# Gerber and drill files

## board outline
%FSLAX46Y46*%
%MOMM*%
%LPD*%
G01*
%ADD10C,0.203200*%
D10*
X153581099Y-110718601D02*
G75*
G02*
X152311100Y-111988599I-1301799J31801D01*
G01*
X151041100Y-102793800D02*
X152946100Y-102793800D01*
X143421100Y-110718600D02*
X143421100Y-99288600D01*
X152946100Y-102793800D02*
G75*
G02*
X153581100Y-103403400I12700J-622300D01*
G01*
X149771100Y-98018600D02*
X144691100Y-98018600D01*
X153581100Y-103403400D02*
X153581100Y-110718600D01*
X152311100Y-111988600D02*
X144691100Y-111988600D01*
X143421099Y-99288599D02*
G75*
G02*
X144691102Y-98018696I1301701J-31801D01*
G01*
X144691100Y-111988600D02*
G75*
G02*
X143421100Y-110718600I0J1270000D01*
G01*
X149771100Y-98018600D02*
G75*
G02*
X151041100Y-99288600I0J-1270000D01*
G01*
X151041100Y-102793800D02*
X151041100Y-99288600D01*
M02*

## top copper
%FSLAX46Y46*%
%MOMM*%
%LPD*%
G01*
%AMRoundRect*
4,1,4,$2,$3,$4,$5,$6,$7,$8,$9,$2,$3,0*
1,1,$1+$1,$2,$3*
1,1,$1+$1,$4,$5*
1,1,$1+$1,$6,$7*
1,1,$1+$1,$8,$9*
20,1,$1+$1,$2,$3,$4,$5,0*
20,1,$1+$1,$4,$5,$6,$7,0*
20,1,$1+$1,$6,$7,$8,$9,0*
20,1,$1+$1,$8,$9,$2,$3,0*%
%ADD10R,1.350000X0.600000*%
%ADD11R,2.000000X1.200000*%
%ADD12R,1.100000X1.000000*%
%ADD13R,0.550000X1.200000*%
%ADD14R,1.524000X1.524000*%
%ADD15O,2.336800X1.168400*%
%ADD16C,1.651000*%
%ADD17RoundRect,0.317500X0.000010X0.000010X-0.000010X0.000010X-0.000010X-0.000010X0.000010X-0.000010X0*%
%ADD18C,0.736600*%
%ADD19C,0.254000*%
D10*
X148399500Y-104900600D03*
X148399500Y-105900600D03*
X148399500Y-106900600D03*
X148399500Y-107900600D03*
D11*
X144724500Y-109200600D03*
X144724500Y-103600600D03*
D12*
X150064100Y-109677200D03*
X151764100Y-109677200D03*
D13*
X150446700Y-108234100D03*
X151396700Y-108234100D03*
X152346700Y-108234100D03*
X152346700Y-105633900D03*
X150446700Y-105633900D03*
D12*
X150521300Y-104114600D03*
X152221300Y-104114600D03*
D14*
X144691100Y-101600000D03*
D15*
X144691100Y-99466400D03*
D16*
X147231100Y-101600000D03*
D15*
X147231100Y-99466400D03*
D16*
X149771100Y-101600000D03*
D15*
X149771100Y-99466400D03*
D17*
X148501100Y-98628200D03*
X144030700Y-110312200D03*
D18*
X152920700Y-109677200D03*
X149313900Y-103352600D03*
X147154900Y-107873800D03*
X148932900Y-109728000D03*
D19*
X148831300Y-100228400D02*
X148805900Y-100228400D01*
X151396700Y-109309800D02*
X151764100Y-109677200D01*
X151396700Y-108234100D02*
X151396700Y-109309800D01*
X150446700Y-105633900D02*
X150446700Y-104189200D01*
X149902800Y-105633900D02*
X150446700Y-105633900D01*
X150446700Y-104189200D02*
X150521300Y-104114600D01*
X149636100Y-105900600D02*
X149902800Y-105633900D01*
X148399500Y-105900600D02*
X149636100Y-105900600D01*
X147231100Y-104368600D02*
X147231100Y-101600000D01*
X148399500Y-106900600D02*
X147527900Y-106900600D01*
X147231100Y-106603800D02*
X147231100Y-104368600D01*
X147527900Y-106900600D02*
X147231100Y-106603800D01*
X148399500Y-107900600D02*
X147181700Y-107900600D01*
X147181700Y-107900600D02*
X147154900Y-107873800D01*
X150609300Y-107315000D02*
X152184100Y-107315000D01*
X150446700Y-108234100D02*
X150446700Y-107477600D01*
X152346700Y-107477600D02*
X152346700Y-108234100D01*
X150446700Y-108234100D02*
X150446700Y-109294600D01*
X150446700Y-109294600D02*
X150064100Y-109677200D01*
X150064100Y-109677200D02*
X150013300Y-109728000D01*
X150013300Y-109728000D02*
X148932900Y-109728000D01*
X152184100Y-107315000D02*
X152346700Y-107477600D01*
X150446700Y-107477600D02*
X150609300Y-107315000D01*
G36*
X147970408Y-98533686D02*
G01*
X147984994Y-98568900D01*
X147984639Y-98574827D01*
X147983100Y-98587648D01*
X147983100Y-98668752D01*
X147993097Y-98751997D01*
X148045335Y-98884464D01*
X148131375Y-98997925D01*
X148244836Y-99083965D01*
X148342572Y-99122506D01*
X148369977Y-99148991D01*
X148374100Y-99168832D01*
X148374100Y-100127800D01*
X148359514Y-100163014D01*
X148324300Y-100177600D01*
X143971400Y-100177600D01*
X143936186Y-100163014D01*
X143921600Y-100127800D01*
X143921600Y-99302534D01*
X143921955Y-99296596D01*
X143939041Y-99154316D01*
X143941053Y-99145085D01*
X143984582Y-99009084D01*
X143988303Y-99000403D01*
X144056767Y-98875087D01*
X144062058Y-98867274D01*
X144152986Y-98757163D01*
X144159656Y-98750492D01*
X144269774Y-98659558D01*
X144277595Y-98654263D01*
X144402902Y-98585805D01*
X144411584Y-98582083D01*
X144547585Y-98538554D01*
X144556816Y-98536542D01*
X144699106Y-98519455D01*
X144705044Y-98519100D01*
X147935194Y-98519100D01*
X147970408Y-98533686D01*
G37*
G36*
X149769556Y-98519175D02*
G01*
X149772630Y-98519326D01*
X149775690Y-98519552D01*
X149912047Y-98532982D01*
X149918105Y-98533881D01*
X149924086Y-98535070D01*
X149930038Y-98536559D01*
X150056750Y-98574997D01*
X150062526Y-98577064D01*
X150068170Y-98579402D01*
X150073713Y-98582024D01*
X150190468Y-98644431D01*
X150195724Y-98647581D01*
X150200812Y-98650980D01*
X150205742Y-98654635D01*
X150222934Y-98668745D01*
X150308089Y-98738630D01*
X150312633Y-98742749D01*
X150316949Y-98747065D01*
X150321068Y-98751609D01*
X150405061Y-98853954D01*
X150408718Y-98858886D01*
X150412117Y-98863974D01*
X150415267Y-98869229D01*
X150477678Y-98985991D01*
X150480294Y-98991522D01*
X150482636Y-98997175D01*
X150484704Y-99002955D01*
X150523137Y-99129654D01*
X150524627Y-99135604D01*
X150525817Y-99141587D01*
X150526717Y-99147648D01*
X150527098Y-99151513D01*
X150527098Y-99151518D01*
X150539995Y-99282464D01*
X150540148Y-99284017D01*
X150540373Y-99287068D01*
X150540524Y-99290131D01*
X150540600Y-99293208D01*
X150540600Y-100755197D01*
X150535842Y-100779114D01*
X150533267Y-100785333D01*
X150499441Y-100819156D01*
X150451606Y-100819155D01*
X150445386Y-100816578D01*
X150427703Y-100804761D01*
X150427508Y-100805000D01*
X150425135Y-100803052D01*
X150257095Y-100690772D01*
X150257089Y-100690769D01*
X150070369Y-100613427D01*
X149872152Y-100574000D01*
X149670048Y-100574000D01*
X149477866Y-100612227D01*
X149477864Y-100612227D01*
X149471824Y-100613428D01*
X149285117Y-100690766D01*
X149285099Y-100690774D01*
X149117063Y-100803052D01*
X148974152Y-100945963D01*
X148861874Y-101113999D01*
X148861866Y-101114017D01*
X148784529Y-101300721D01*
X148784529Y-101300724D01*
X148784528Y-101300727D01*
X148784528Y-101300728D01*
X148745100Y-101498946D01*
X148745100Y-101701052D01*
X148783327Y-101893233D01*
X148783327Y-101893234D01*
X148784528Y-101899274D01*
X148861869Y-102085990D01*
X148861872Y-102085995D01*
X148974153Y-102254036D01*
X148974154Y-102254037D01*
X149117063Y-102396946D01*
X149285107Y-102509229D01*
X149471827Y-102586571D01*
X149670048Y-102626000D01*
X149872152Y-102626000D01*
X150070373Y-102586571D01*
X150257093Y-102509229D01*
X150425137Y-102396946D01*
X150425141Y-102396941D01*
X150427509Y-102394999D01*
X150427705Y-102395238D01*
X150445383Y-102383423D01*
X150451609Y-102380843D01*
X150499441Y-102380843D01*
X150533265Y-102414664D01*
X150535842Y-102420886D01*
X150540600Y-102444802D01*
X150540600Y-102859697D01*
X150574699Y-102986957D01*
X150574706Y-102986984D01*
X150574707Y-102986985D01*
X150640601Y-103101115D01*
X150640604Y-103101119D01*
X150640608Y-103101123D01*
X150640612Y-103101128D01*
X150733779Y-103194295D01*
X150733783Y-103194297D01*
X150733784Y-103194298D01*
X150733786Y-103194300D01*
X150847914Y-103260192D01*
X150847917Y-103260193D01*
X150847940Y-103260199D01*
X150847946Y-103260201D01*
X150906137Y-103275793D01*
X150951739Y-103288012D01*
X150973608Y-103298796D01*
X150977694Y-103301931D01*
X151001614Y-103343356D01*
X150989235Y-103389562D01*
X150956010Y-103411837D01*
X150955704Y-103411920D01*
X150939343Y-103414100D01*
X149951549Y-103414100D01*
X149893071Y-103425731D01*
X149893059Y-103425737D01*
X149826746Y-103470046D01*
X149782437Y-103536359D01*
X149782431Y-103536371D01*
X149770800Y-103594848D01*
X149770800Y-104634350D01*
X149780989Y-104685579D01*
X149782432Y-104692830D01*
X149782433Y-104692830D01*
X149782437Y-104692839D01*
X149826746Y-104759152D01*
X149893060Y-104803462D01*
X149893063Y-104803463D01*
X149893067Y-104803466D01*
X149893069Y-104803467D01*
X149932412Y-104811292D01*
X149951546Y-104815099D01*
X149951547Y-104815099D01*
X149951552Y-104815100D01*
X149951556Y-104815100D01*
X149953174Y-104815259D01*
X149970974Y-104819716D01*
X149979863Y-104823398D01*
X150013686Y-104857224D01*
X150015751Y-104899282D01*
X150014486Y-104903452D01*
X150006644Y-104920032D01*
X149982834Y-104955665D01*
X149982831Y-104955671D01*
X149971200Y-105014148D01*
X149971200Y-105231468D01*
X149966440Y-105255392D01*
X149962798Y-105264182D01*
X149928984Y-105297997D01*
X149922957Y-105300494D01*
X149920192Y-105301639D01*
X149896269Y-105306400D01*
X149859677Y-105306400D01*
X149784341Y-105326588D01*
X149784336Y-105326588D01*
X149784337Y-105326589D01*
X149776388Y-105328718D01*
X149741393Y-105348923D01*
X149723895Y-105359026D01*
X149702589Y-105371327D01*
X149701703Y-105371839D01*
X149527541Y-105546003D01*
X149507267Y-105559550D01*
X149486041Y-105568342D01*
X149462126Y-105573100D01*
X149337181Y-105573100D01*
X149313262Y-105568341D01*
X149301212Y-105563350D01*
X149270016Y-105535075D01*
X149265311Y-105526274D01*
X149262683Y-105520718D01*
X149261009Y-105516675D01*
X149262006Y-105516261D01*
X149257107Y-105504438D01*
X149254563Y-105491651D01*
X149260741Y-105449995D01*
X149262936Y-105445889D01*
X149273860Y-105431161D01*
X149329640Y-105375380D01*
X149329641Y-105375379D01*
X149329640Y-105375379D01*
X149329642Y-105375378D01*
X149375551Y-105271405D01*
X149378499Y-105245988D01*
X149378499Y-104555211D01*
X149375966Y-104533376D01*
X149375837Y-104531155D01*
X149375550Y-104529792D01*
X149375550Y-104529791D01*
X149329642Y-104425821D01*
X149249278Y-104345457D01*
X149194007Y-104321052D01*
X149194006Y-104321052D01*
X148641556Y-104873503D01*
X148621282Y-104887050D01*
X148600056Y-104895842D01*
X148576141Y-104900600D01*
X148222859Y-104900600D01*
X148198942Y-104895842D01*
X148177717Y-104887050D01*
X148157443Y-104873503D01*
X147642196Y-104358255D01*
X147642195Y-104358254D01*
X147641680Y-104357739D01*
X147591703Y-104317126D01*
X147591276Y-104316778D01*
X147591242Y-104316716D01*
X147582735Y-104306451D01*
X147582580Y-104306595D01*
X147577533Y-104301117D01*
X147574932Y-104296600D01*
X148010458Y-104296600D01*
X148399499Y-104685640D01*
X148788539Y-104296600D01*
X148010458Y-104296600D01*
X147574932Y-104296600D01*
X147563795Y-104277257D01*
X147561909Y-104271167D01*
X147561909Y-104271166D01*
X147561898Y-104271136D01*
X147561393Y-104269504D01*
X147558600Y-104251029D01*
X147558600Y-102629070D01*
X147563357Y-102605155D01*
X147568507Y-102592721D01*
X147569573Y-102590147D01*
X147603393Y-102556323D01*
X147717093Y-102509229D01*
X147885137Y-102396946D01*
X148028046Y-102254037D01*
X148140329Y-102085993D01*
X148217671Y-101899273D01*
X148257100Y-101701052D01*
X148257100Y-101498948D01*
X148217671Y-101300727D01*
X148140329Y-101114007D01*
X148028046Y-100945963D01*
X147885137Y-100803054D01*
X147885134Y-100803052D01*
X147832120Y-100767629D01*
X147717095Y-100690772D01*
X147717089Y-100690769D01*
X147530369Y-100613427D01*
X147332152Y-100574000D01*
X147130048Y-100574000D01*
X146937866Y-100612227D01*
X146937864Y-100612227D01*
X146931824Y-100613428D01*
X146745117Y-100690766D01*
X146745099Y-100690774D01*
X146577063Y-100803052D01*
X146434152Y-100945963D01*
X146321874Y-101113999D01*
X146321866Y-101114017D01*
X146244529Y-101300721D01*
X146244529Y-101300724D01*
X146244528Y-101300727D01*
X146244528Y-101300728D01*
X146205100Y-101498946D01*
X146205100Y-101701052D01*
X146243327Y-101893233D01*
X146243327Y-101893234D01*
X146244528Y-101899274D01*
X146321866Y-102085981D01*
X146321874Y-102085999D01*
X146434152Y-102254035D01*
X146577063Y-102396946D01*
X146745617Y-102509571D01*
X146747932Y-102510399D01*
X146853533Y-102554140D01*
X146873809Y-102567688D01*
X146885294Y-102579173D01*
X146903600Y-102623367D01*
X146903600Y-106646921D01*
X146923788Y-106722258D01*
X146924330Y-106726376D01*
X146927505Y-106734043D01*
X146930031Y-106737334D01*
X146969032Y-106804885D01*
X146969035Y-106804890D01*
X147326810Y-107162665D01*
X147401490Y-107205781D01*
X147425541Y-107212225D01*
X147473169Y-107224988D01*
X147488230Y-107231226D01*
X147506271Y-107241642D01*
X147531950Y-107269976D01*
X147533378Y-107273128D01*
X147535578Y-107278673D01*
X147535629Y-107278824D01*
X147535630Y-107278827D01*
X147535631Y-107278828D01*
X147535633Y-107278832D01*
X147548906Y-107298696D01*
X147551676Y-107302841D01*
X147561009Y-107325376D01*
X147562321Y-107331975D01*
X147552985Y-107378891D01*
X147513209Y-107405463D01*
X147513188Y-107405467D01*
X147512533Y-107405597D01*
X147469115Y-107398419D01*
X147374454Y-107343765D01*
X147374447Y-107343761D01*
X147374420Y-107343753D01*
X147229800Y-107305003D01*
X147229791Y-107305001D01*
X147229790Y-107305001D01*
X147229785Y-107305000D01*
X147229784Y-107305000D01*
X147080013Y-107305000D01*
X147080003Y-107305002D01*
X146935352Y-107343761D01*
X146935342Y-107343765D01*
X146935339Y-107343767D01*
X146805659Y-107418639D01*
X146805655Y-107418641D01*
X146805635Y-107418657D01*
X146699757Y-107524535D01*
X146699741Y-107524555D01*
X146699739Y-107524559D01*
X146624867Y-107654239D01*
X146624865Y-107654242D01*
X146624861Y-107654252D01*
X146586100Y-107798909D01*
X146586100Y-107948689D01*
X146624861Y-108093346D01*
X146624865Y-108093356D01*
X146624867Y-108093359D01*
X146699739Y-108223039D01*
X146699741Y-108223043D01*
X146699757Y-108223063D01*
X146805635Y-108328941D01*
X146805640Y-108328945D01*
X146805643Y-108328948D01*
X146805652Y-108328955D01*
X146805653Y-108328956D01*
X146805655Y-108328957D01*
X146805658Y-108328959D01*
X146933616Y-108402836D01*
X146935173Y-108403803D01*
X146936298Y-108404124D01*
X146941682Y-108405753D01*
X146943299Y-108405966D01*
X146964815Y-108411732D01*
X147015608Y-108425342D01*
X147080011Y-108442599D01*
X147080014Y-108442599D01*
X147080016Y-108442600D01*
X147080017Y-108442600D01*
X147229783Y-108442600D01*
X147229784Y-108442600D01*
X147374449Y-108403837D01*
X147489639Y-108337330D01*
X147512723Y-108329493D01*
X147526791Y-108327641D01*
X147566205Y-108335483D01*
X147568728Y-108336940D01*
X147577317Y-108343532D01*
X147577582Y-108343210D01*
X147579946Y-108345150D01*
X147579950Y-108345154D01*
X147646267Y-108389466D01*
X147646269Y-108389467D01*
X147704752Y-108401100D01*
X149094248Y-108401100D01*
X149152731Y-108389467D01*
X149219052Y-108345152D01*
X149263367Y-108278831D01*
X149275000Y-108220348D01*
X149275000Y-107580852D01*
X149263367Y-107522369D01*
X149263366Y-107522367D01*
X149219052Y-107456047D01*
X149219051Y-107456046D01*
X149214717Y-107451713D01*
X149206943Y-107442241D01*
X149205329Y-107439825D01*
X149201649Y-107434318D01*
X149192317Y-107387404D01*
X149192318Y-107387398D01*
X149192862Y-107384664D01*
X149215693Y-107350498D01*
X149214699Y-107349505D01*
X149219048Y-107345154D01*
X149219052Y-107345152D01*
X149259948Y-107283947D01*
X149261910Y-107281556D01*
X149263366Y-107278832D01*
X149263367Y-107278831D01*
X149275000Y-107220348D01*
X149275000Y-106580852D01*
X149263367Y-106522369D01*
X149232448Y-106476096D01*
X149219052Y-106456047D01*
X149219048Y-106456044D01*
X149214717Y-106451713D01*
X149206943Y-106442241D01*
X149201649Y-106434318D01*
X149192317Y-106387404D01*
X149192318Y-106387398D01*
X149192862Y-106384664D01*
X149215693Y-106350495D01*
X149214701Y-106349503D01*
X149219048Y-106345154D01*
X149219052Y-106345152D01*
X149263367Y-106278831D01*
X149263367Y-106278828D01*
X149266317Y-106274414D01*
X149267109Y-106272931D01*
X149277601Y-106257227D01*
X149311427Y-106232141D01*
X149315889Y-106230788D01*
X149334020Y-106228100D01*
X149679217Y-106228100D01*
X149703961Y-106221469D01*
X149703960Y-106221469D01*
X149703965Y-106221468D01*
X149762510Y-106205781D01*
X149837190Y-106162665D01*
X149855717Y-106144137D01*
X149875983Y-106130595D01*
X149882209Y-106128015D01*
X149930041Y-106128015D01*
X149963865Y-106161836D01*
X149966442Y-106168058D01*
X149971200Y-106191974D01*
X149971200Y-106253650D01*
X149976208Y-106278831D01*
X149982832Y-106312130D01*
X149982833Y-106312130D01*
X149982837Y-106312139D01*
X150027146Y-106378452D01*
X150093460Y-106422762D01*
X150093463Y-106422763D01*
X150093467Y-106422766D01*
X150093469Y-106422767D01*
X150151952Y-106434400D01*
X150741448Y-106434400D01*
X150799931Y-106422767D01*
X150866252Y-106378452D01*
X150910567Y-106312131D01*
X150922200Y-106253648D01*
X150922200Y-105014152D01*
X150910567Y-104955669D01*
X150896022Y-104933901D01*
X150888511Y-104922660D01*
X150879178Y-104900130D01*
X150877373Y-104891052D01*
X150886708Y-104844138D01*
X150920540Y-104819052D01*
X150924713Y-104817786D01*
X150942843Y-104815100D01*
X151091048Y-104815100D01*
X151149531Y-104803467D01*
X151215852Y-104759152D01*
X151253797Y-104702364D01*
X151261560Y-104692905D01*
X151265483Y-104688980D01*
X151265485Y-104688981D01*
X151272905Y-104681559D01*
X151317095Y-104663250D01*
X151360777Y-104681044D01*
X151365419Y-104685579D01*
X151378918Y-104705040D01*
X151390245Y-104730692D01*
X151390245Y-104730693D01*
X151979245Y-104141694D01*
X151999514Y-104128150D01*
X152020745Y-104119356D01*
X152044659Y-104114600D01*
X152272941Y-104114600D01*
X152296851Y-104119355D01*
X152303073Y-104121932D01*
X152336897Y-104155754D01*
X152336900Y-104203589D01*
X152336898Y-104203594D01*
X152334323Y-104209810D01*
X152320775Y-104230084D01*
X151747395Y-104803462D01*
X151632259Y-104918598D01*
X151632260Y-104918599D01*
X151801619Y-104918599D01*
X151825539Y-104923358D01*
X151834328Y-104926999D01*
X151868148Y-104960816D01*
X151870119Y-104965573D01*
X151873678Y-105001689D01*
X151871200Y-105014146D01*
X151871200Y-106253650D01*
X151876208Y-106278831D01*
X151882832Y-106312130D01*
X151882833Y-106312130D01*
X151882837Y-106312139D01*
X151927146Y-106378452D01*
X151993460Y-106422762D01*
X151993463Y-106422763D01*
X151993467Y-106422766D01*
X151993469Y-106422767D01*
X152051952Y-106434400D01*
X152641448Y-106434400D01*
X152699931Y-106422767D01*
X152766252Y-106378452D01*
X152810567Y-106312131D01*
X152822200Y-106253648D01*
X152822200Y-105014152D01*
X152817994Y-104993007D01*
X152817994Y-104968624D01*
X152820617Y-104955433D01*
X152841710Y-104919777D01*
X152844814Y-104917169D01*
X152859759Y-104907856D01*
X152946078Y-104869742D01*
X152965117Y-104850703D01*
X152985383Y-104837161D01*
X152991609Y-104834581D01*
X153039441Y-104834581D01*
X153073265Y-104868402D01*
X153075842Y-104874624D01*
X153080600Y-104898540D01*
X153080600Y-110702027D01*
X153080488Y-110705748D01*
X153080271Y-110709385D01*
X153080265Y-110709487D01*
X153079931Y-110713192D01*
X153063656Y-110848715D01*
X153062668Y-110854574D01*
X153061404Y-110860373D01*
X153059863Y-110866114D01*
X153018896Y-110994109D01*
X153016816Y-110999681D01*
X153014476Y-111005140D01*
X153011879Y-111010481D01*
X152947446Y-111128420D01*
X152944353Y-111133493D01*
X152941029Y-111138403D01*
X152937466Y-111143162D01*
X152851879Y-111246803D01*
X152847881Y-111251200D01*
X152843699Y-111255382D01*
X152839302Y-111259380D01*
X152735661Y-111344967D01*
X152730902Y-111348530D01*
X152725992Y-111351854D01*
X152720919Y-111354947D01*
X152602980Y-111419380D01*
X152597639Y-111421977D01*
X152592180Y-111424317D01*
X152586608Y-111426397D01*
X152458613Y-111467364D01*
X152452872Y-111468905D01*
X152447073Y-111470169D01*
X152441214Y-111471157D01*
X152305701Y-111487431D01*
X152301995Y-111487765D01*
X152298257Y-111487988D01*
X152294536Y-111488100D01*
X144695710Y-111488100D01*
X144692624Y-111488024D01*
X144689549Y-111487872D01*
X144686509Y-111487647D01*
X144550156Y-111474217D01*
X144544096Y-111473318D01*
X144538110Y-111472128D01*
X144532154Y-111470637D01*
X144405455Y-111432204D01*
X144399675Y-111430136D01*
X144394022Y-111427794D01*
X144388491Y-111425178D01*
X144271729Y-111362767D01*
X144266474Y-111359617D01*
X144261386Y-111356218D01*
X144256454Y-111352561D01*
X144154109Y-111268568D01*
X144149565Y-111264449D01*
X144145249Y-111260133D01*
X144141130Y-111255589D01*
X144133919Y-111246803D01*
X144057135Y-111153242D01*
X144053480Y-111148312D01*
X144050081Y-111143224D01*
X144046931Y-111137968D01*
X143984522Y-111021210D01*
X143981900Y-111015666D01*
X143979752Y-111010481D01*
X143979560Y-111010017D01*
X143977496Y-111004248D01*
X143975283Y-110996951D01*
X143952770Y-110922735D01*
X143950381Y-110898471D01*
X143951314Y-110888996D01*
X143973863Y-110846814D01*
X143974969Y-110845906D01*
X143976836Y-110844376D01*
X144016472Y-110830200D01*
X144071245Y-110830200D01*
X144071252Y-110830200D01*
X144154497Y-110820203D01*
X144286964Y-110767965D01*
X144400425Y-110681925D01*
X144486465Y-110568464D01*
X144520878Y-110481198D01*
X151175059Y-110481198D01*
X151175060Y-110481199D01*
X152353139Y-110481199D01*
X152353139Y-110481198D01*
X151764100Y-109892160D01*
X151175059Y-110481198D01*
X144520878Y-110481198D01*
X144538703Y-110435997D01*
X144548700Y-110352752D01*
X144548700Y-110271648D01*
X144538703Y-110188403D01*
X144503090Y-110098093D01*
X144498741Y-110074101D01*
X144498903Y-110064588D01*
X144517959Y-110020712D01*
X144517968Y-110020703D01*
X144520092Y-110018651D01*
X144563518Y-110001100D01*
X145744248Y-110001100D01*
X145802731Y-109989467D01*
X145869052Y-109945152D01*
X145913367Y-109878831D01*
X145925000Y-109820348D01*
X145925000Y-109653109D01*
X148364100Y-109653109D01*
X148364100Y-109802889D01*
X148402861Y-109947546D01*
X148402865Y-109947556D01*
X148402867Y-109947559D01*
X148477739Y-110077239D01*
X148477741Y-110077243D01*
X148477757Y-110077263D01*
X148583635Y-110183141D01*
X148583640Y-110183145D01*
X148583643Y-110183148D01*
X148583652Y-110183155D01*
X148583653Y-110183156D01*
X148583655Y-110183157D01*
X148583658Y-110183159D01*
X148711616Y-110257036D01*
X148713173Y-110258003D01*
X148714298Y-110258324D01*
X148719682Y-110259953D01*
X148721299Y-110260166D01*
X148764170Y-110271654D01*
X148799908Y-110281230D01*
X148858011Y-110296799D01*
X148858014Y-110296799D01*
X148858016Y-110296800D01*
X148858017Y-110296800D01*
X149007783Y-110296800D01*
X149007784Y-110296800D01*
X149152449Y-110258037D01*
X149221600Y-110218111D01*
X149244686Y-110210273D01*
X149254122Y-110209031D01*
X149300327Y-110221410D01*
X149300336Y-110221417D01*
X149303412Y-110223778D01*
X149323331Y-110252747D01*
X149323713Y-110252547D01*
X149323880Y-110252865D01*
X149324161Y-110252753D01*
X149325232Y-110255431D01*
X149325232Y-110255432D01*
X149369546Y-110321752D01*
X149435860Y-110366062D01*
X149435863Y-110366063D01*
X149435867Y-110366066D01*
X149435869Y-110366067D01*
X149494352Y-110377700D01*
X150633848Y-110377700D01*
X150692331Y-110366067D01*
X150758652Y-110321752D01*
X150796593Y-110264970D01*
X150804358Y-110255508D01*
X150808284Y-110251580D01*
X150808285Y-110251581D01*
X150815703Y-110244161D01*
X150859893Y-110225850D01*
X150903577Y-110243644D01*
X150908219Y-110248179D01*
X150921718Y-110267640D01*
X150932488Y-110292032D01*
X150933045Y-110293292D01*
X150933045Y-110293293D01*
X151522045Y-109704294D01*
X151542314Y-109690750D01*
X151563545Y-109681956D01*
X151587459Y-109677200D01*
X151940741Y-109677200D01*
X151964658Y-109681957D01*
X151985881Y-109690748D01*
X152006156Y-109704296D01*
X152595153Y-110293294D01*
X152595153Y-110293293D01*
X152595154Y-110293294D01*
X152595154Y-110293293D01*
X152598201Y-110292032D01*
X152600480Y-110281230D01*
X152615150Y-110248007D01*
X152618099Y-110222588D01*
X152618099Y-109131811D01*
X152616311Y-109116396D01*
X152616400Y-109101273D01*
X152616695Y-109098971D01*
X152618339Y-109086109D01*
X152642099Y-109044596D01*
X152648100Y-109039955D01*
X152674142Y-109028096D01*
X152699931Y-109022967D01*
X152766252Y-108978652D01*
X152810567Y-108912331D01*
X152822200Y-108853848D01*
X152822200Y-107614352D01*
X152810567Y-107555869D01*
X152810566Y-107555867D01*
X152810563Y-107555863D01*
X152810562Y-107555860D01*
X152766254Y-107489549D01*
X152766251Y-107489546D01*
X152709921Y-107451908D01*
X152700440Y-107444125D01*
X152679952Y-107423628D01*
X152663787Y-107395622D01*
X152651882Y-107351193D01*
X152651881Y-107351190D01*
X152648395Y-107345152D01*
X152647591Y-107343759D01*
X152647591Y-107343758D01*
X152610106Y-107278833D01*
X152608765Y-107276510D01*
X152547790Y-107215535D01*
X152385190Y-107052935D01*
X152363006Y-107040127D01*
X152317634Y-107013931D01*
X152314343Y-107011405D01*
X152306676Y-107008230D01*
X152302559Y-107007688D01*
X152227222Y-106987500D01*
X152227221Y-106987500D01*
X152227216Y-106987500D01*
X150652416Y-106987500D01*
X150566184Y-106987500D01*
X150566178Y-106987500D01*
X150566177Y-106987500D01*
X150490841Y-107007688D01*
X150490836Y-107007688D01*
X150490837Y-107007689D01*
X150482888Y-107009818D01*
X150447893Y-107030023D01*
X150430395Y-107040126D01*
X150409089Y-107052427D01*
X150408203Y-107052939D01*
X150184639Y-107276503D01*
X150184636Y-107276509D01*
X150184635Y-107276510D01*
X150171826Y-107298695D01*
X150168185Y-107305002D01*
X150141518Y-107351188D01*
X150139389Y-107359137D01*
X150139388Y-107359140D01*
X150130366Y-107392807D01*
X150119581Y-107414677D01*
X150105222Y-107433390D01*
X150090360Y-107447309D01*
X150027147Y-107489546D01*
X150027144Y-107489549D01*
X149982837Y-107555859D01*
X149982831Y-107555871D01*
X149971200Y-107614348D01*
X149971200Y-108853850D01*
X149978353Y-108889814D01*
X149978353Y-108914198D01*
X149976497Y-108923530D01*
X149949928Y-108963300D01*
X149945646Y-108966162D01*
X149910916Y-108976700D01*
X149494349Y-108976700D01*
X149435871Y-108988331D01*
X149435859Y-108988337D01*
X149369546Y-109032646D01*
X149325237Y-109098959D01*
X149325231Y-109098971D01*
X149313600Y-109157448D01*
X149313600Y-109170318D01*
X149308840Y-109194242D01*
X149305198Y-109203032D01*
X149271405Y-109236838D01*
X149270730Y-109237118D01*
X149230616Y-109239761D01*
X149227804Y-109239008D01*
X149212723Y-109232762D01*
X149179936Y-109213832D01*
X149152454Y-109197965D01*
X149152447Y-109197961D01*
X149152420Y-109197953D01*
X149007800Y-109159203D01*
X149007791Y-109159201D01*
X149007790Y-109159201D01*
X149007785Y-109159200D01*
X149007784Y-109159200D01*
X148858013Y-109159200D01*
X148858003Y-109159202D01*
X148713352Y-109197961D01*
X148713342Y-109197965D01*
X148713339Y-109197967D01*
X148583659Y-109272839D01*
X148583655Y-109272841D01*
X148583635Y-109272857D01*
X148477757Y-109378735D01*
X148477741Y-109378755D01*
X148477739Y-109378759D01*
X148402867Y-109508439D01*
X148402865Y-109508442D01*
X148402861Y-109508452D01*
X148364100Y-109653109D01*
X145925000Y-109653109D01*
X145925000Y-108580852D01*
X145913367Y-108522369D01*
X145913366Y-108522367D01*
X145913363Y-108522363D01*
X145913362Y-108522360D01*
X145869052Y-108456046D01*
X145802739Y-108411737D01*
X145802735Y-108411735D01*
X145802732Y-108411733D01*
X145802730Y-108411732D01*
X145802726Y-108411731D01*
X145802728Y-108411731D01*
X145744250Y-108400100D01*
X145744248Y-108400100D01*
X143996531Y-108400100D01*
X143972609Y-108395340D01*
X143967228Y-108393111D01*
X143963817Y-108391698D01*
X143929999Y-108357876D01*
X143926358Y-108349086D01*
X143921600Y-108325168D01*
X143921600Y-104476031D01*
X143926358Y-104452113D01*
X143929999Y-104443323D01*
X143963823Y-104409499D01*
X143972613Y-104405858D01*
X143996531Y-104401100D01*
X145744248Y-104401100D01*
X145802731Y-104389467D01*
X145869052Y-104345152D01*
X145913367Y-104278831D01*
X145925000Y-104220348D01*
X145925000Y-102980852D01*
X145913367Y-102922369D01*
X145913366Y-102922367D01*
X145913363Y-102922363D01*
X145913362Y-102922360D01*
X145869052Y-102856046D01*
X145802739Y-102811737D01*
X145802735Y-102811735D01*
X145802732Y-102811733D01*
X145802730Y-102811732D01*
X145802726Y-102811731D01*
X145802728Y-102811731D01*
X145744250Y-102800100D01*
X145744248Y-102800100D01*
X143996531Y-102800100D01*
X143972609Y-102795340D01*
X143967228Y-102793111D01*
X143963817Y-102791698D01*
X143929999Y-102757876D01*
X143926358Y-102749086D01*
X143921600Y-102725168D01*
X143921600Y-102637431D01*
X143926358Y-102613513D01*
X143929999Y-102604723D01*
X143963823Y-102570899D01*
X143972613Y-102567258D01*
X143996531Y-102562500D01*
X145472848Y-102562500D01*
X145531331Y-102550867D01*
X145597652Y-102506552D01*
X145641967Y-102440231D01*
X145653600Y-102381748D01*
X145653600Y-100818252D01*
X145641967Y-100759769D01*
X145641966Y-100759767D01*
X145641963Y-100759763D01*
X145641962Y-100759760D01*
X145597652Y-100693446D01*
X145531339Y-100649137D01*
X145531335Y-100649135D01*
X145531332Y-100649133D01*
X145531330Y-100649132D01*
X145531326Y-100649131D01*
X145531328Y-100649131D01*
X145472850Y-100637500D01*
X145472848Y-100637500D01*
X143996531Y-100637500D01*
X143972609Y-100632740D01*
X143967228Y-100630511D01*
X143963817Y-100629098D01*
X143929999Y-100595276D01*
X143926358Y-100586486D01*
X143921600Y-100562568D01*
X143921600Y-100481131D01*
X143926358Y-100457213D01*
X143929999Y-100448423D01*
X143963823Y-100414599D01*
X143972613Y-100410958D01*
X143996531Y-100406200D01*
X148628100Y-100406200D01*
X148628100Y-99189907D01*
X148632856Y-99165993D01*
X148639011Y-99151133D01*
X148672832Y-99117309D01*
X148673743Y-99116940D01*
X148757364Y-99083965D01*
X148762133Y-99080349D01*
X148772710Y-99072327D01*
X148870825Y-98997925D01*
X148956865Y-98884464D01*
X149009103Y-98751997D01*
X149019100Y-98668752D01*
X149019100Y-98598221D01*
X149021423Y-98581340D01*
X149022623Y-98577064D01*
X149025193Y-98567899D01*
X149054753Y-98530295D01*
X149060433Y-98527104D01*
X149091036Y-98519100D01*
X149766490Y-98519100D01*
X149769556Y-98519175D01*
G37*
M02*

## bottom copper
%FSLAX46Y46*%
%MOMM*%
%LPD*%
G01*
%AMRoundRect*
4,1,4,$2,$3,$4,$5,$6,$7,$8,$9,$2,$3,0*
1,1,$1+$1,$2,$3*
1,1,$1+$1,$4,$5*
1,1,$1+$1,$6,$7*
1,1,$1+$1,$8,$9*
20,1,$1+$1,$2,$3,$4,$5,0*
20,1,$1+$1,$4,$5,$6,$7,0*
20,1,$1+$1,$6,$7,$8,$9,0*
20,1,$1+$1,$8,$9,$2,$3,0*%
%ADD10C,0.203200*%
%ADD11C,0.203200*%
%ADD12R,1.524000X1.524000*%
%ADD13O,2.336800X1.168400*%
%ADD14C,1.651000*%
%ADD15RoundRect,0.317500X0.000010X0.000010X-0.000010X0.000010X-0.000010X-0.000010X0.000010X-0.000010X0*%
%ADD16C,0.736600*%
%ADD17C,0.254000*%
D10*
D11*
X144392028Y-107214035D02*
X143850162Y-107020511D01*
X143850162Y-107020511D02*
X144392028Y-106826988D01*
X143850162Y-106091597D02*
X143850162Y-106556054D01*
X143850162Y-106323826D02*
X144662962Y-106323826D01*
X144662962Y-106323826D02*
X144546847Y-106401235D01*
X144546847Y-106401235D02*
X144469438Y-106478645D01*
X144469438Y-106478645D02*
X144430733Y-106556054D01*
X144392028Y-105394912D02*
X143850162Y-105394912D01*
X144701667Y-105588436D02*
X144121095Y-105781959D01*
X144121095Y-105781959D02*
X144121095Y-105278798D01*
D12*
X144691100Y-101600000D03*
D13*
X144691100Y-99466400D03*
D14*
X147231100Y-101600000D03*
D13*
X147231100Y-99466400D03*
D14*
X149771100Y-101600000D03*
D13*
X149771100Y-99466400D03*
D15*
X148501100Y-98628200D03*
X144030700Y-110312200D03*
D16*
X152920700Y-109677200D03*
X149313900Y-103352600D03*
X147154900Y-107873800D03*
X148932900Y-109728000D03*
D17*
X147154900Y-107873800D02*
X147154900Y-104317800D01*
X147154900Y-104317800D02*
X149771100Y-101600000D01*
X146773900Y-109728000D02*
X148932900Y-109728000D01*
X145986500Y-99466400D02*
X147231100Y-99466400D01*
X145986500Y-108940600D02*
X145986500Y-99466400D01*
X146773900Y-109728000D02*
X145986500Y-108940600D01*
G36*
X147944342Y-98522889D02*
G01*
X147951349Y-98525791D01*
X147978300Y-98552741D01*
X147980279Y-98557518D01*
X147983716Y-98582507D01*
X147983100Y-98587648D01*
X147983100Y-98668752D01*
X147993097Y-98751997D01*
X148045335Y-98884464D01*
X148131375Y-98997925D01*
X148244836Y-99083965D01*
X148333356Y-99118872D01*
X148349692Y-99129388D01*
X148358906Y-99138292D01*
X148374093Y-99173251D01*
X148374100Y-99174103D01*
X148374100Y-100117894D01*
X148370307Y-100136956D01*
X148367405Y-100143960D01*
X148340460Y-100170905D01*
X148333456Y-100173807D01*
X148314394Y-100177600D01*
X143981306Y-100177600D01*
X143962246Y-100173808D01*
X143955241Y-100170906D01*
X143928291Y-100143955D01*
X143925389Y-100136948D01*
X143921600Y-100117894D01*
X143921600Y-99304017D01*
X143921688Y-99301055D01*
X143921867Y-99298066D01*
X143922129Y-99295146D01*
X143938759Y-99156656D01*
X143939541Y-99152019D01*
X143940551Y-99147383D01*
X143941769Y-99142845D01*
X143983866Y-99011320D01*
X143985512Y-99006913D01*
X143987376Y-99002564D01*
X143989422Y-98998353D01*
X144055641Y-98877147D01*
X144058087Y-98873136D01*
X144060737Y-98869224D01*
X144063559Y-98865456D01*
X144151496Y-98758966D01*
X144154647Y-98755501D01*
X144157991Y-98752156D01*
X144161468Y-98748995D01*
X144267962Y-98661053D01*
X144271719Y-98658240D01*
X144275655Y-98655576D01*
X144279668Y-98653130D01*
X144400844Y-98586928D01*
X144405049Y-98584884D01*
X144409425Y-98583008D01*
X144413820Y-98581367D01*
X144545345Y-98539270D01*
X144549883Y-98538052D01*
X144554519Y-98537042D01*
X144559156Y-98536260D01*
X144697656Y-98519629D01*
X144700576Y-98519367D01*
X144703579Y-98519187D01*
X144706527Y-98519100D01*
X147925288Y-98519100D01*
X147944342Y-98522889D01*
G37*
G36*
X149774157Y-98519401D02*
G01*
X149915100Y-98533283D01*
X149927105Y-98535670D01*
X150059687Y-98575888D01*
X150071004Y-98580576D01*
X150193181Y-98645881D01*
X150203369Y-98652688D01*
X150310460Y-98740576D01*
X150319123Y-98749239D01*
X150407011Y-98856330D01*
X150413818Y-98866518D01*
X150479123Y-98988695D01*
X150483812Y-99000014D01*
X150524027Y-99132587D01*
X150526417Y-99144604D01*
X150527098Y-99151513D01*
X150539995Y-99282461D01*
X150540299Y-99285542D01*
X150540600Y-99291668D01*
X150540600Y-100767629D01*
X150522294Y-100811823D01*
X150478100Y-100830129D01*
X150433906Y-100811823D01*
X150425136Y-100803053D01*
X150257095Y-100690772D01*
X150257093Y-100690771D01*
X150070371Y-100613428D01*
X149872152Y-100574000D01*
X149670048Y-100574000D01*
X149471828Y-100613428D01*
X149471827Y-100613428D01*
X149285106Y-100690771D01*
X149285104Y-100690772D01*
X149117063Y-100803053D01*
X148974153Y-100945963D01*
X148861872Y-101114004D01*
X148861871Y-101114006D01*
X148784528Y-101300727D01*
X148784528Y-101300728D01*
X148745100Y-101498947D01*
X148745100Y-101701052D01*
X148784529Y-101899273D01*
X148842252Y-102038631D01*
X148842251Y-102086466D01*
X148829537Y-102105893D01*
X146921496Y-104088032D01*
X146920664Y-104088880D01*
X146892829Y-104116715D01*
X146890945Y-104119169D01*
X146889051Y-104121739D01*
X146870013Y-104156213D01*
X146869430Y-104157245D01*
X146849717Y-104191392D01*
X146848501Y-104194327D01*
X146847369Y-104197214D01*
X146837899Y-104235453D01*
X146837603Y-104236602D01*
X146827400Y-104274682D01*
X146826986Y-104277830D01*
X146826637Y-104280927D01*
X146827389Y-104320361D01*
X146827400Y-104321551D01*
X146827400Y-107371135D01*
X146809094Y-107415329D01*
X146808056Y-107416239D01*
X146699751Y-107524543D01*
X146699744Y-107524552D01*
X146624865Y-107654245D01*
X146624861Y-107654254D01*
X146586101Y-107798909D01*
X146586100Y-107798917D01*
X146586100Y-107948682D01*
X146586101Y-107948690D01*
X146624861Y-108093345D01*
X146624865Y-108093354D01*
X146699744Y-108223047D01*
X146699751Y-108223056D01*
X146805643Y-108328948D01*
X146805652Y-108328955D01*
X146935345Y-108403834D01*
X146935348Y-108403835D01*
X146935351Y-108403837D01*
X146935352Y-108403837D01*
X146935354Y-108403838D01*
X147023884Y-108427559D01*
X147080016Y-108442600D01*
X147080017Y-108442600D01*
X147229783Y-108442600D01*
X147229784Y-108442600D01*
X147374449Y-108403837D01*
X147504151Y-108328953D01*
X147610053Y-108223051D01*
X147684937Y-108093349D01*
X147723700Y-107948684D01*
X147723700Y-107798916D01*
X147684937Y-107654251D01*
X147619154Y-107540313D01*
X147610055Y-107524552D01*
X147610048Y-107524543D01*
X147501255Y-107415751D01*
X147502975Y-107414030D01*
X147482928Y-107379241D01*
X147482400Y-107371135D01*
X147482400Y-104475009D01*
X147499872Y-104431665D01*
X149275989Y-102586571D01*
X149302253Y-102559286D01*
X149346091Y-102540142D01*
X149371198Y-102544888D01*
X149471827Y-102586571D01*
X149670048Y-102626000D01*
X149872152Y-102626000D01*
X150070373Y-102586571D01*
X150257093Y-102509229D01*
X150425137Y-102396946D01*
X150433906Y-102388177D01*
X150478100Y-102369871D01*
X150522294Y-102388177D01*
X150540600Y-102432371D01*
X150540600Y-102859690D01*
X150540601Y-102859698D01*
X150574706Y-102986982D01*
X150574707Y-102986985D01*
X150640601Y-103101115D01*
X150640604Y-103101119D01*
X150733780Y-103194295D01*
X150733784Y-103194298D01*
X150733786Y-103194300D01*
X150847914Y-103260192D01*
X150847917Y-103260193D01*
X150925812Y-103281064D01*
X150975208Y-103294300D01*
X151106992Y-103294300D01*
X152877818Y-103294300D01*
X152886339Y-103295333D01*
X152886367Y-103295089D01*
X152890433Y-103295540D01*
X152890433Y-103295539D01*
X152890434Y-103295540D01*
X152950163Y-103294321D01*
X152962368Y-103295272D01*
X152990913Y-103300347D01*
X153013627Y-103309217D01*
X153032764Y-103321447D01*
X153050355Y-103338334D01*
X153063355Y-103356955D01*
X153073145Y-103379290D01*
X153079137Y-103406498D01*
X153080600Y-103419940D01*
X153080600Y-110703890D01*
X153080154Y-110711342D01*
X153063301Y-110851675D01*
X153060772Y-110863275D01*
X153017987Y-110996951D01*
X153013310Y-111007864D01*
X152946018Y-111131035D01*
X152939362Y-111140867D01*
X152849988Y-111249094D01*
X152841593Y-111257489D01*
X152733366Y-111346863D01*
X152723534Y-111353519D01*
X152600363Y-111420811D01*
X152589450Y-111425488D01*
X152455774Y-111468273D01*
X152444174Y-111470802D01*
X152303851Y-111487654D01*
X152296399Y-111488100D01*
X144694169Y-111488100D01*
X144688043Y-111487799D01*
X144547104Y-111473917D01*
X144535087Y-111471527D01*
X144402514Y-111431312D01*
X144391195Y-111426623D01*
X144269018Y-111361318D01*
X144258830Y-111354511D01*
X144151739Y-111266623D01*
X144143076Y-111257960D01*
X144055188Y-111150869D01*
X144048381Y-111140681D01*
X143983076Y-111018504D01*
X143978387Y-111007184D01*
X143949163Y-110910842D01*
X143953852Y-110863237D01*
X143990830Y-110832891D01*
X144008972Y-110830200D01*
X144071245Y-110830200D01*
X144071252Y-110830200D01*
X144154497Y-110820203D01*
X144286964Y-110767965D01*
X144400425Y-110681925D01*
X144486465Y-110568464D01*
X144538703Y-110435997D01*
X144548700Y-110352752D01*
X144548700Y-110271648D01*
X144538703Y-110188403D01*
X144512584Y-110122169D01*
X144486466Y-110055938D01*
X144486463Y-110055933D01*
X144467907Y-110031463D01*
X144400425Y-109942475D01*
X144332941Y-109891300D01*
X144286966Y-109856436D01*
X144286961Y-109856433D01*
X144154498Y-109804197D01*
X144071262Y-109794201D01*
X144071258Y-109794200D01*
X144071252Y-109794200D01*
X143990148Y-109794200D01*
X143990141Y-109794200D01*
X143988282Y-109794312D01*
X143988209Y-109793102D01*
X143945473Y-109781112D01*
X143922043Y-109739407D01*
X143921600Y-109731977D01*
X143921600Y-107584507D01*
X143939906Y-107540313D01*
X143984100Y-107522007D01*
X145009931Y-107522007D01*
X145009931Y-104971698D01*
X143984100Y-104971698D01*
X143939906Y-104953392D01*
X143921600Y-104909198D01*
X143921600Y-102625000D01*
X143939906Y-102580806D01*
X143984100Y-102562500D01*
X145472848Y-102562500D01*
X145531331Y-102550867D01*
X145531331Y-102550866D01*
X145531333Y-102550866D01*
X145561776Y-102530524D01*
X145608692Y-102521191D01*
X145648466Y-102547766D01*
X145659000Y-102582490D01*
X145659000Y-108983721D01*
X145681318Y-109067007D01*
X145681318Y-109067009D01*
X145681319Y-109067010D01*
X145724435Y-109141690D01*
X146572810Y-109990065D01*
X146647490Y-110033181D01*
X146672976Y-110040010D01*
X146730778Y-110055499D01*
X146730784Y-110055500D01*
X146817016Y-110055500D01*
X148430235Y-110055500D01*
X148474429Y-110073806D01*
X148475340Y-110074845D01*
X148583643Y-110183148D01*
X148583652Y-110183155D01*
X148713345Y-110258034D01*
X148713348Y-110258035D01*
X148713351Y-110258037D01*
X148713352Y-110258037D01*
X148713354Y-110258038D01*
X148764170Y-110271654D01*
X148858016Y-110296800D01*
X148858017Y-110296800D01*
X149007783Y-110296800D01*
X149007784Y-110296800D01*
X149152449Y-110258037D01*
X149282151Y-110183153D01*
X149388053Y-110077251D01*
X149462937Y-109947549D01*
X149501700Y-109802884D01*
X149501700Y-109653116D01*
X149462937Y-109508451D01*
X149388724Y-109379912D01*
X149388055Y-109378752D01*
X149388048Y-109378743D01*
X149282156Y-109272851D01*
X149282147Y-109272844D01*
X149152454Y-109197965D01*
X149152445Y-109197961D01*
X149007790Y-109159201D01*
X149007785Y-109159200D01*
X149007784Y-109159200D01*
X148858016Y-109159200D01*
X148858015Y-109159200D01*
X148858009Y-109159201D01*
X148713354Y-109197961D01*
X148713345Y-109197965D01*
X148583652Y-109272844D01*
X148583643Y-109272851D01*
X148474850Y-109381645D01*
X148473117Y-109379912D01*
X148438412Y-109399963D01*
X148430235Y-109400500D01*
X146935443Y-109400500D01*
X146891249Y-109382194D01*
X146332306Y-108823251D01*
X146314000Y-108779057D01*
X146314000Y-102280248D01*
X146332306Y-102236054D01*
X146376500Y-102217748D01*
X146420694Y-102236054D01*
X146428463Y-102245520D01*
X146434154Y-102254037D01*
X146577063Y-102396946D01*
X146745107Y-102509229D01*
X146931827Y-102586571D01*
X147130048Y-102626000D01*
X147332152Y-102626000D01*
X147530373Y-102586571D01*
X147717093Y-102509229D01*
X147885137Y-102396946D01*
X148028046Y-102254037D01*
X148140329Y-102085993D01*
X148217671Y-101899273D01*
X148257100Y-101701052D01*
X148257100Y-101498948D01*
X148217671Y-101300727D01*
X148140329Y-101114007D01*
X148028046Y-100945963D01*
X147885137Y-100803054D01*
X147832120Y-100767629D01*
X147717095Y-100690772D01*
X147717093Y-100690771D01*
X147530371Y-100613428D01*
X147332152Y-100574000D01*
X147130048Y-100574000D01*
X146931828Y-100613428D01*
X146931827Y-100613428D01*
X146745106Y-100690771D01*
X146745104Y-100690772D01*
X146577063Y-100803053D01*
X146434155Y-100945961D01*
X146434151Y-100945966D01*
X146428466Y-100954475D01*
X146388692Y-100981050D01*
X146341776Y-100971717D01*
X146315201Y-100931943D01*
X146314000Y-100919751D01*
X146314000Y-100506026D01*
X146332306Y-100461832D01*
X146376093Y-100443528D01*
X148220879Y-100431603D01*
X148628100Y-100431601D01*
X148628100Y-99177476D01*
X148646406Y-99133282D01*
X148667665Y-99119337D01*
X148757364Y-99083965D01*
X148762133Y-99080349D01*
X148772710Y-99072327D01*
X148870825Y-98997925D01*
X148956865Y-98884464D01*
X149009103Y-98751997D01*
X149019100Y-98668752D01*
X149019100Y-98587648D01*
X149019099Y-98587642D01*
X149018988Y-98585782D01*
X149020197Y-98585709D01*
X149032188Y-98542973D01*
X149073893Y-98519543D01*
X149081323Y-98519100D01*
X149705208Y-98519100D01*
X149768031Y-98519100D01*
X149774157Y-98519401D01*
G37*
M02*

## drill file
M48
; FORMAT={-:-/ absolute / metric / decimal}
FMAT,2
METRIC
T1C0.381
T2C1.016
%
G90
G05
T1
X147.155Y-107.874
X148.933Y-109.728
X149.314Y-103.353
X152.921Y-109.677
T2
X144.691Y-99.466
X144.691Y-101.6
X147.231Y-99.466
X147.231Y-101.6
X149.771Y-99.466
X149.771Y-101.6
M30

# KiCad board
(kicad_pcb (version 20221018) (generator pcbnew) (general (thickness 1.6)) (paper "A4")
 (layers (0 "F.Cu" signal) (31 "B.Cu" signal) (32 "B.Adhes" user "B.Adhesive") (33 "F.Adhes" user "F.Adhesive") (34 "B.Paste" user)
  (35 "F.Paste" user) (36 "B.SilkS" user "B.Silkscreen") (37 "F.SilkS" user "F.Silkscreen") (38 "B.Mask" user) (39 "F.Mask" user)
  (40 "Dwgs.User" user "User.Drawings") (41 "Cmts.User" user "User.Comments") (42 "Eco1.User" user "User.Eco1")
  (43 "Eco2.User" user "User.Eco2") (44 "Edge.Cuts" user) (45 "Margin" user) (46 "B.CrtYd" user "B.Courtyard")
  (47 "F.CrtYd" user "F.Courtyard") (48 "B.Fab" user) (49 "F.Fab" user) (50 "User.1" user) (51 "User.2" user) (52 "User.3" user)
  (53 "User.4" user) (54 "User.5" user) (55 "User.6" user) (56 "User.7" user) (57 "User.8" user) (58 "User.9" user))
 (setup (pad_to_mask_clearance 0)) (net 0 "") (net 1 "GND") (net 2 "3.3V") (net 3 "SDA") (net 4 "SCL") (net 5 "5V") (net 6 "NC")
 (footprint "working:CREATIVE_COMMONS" (layer "F.Cu") (at 131.9911 125.9586)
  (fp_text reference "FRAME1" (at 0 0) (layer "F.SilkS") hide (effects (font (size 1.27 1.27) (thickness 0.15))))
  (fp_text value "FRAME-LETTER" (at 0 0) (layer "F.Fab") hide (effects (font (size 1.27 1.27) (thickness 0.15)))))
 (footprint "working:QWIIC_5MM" (layer "F.Cu") (at 146.8501 110.8456)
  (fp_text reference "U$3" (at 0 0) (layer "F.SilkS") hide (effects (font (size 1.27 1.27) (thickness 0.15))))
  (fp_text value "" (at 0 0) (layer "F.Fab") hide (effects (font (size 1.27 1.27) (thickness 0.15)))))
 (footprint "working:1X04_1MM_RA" (layer "F.Cu") (at 148.3995 106.4006 -90)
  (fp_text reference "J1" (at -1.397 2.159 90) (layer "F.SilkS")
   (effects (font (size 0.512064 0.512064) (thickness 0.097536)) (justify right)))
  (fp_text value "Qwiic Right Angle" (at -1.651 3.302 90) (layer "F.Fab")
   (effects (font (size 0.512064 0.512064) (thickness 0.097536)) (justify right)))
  (pad "1" smd rect (at -1.5 0 270) (size 0.6 1.35) (layers "F.Cu" "F.Paste" "F.Mask") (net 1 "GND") (solder_mask_margin 0.1016)
   (thermal_bridge_angle 45))
  (pad "2" smd rect (at -0.5 0 270) (size 0.6 1.35) (layers "F.Cu" "F.Paste" "F.Mask") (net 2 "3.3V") (solder_mask_margin 0.1016)
   (thermal_bridge_angle 45))
  (pad "3" smd rect (at 0.5 0 270) (size 0.6 1.35) (layers "F.Cu" "F.Paste" "F.Mask") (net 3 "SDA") (solder_mask_margin 0.1016)
   (thermal_bridge_angle 45))
  (pad "4" smd rect (at 1.5 0 270) (size 0.6 1.35) (layers "F.Cu" "F.Paste" "F.Mask") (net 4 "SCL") (solder_mask_margin 0.1016)
   (thermal_bridge_angle 45))
  (pad "NC1" smd rect (at 2.8 3.675 270) (size 1.2 2) (layers "F.Cu" "F.Paste" "F.Mask") (solder_mask_margin 0.1016)
   (thermal_bridge_angle 45))
  (pad "NC2" smd rect (at -2.8 3.675 270) (size 1.2 2) (layers "F.Cu" "F.Paste" "F.Mask") (solder_mask_margin 0.1016)
   (thermal_bridge_angle 45)))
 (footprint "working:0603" (layer "F.Cu") (at 150.9141 109.6772)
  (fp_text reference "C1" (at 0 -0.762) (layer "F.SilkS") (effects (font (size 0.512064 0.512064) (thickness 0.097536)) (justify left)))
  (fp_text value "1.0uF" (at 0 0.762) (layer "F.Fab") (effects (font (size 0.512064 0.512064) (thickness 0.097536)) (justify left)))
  (pad "1" smd rect (at -0.85 0) (size 1.1 1) (layers "F.Cu" "F.Paste" "F.Mask") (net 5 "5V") (solder_mask_margin 0.1016)
   (thermal_bridge_angle 45))
  (pad "2" smd rect (at 0.85 0) (size 1.1 1) (layers "F.Cu" "F.Paste" "F.Mask") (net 1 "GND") (solder_mask_margin 0.1016)
   (thermal_bridge_angle 45)))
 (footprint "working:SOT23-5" (layer "F.Cu") (at 151.3967 106.934)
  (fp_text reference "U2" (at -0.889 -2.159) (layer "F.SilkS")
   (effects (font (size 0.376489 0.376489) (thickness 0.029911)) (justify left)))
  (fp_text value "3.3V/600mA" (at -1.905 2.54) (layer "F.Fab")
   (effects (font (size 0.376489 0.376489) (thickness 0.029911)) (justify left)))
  (pad "1" smd rect (at -0.95 1.3001) (size 0.55 1.2) (layers "F.Cu" "F.Paste" "F.Mask") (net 5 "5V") (solder_mask_margin 0.1016)
   (thermal_bridge_angle 45))
  (pad "2" smd rect (at 0 1.3001) (size 0.55 1.2) (layers "F.Cu" "F.Paste" "F.Mask") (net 1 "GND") (solder_mask_margin 0.1016)
   (thermal_bridge_angle 45))
  (pad "3" smd rect (at 0.95 1.3001) (size 0.55 1.2) (layers "F.Cu" "F.Paste" "F.Mask") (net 5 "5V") (solder_mask_margin 0.1016)
   (thermal_bridge_angle 45))
  (pad "4" smd rect (at 0.95 -1.3001) (size 0.55 1.2) (layers "F.Cu" "F.Paste" "F.Mask") (solder_mask_margin 0.1016)
   (thermal_bridge_angle 45))
  (pad "5" smd rect (at -0.95 -1.3001) (size 0.55 1.2) (layers "F.Cu" "F.Paste" "F.Mask") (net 2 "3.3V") (solder_mask_margin 0.1016)
   (thermal_bridge_angle 45)))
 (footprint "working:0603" (layer "F.Cu") (at 151.3713 104.1146)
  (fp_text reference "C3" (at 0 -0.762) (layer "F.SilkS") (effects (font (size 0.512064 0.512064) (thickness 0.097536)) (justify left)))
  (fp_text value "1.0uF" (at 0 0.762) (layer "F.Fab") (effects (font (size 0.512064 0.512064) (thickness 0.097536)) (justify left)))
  (pad "1" smd rect (at -0.85 0) (size 1.1 1) (layers "F.Cu" "F.Paste" "F.Mask") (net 2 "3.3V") (solder_mask_margin 0.1016)
   (thermal_bridge_angle 45))
  (pad "2" smd rect (at 0.85 0) (size 1.1 1) (layers "F.Cu" "F.Paste" "F.Mask") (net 1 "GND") (solder_mask_margin 0.1016)
   (thermal_bridge_angle 45)))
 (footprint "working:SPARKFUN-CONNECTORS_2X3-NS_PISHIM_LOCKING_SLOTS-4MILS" (layer "F.Cu") (at 147.2311 100.5586)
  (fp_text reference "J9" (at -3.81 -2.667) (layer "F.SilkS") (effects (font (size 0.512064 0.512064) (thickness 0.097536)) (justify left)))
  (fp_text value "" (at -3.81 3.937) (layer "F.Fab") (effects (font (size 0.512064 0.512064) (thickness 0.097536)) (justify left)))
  (pad "1" thru_hole rect (at -2.54 1.0414) (size 1.524 1.524) (drill 1.016) (layers "*.Cu" "*.Mask") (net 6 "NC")
   (solder_mask_margin 0.1016) (thermal_bridge_angle 45))
  (pad "2" thru_hole oval (at -2.54 -1.0922) (size 2.3368 1.1684) (drill 1.016) (layers "*.Cu") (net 5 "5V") (solder_mask_margin 0.1016)
   (zone_connect 2) (thermal_bridge_angle 45))
  (pad "3" thru_hole circle (at 0 1.0414) (size 1.651 1.651) (drill 1.016) (layers "*.Cu" "*.Mask") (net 3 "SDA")
   (solder_mask_margin 0.1016))
  (pad "4" thru_hole oval (at 0 -1.0922) (size 2.3368 1.1684) (drill 1.016) (layers "*.Cu") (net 5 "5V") (solder_mask_margin 0.1016)
   (zone_connect 2) (thermal_bridge_angle 45))
  (pad "5" thru_hole circle (at 2.54 1.0414) (size 1.651 1.651) (drill 1.016) (layers "*.Cu" "*.Mask") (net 4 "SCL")
   (solder_mask_margin 0.1016))
  (pad "6" thru_hole oval (at 2.54 -1.0922) (size 2.3368 1.1684) (drill 1.016) (layers "*.Cu") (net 1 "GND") (solder_mask_margin 0.1016)
   (zone_connect 2) (thermal_bridge_angle 45)))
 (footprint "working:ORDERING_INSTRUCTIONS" (layer "F.Cu") (at 111.6711 127.2286)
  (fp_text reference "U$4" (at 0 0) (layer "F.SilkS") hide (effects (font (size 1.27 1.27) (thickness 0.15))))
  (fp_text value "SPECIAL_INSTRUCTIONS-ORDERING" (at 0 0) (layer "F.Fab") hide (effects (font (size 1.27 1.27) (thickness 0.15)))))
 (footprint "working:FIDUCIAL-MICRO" (layer "F.Cu") (at 148.5011 98.6282 180)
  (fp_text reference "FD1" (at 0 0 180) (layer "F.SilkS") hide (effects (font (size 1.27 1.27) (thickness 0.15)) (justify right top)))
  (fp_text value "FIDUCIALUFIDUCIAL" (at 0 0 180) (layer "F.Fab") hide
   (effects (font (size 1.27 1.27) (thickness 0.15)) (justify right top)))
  (pad "1" smd roundrect (at 0 0 180) (size 0.635 0.635) (layers "F.Cu" "F.Mask") (roundrect_rratio 0.5) (solder_mask_margin 0.1016)
   (thermal_bridge_angle 45)))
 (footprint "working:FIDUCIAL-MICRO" (layer "F.Cu") (at 144.0307 110.3122 180)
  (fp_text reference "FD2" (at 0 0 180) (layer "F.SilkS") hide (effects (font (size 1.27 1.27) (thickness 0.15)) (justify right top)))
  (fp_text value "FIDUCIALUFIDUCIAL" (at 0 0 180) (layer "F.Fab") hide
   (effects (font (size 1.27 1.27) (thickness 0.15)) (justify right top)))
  (pad "1" smd roundrect (at 0 0 180) (size 0.635 0.635) (layers "F.Cu" "F.Mask") (roundrect_rratio 0.5) (solder_mask_margin 0.1016)
   (thermal_bridge_angle 45)))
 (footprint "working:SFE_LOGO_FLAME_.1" (layer "B.Cu") (at 152.8445 111.633 180)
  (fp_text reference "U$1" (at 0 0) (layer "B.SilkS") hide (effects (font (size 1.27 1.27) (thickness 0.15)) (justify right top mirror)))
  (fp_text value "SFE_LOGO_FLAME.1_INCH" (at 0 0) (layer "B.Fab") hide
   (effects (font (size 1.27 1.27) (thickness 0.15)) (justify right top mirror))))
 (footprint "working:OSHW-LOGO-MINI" (layer "B.Cu") (at 146.0119 110.363 180)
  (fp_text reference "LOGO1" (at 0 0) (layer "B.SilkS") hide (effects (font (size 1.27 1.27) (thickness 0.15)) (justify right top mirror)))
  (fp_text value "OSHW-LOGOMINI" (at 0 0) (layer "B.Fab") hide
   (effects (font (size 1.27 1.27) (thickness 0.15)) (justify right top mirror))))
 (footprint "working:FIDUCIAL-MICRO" (layer "B.Cu") (at 148.5011 98.6282 180)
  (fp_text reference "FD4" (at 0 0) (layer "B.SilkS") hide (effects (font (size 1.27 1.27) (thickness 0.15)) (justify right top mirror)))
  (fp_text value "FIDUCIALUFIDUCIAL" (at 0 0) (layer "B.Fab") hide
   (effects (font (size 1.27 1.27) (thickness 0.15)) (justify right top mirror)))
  (pad "1" smd roundrect (at 0 0 180) (size 0.635 0.635) (layers "B.Cu" "B.Mask") (roundrect_rratio 0.5) (solder_mask_margin 0.1016)
   (thermal_bridge_angle 45)))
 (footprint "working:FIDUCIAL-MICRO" (layer "B.Cu") (at 144.0307 110.3122 180)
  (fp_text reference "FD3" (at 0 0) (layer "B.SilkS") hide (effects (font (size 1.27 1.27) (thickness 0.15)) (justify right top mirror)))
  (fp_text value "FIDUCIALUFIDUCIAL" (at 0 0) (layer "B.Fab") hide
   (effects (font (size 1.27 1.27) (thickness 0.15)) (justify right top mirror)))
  (pad "1" smd roundrect (at 0 0 180) (size 0.635 0.635) (layers "B.Cu" "B.Mask") (roundrect_rratio 0.5) (solder_mask_margin 0.1016)
   (thermal_bridge_angle 45)))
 (gr_arc (start 153.581099 110.718601) (mid 153.200099 111.6076) (end 152.3111 111.9886) (stroke (width 0.2032) (type solid))
  (layer "Edge.Cuts"))
 (gr_line (start 151.0411 102.7938) (end 152.9461 102.7938) (stroke (width 0.2032) (type solid)) (layer "Edge.Cuts"))
 (gr_line (start 143.4211 110.7186) (end 143.4211 99.2886) (stroke (width 0.2032) (type solid)) (layer "Edge.Cuts"))
 (gr_arc (start 152.9461 102.7938) (mid 153.389852 102.967087) (end 153.5811 103.4034) (stroke (width 0.2032) (type solid))
  (layer "Edge.Cuts"))
 (gr_line (start 149.7711 98.0186) (end 144.6911 98.0186) (stroke (width 0.2032) (type solid)) (layer "Edge.Cuts"))
 (gr_line (start 153.5811 103.4034) (end 153.5811 110.7186) (stroke (width 0.2032) (type solid)) (layer "Edge.Cuts"))
 (gr_line (start 152.3111 111.9886) (end 144.6911 111.9886) (stroke (width 0.2032) (type solid)) (layer "Edge.Cuts"))
 (gr_arc (start 143.421099 99.288599) (mid 143.8021 98.399599) (end 144.6911 98.0186) (stroke (width 0.2032) (type solid))
  (layer "Edge.Cuts"))
 (gr_arc (start 144.6911 111.9886) (mid 143.793074 111.616626) (end 143.4211 110.7186) (stroke (width 0.2032) (type solid))
  (layer "Edge.Cuts"))
 (gr_arc (start 149.7711 98.0186) (mid 150.669126 98.390574) (end 151.0411 99.2886) (stroke (width 0.2032) (type solid)) (layer "Edge.Cuts"))
 (gr_line (start 151.0411 102.7938) (end 151.0411 99.2886) (stroke (width 0.2032) (type solid)) (layer "Edge.Cuts"))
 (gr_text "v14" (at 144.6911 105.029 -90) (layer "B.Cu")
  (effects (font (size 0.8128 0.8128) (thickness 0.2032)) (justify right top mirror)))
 (segment (start 148.8313 100.2284) (end 148.8059 100.2284) (width 0.254) (layer "F.Cu") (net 1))
 (segment (start 151.3967 109.3098) (end 151.7641 109.6772) (width 0.254) (layer "F.Cu") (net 1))
 (segment (start 151.3967 108.2341) (end 151.3967 109.3098) (width 0.254) (layer "F.Cu") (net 1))
 (via (at 152.9207 109.6772) (size 0.7366) (drill 0.381) (layers "F.Cu" "B.Cu") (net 1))
 (via (at 149.3139 103.3526) (size 0.7366) (drill 0.381) (layers "F.Cu" "B.Cu") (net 1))
 (segment (start 150.4467 105.6339) (end 150.4467 104.1892) (width 0.254) (layer "F.Cu") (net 2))
 (segment (start 149.9028 105.6339) (end 150.4467 105.6339) (width 0.254) (layer "F.Cu") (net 2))
 (segment (start 150.4467 104.1892) (end 150.5213 104.1146) (width 0.254) (layer "F.Cu") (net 2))
 (segment (start 149.6361 105.9006) (end 149.9028 105.6339) (width 0.254) (layer "F.Cu") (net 2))
 (segment (start 148.3995 105.9006) (end 149.6361 105.9006) (width 0.254) (layer "F.Cu") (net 2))
 (segment (start 147.2311 104.3686) (end 147.2311 101.6) (width 0.254) (layer "F.Cu") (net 3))
 (segment (start 148.3995 106.9006) (end 147.5279 106.9006) (width 0.254) (layer "F.Cu") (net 3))
 (segment (start 147.2311 106.6038) (end 147.2311 104.3686) (width 0.254) (layer "F.Cu") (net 3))
 (segment (start 147.5279 106.9006) (end 147.2311 106.6038) (width 0.254) (layer "F.Cu") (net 3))
 (segment (start 148.3995 107.9006) (end 147.1817 107.9006) (width 0.254) (layer "F.Cu") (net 4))
 (segment (start 147.1817 107.9006) (end 147.1549 107.8738) (width 0.254) (layer "F.Cu") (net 4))
 (via (at 147.1549 107.8738) (size 0.7366) (drill 0.381) (layers "F.Cu" "B.Cu") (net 4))
 (segment (start 147.1549 107.8738) (end 147.1549 104.3178) (width 0.254) (layer "B.Cu") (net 4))
 (segment (start 147.1549 104.3178) (end 149.7711 101.6) (width 0.254) (layer "B.Cu") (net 4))
 (segment (start 150.6093 107.315) (end 152.1841 107.315) (width 0.254) (layer "F.Cu") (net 5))
 (segment (start 150.4467 108.2341) (end 150.4467 107.4776) (width 0.254) (layer "F.Cu") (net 5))
 (segment (start 152.3467 107.4776) (end 152.3467 108.2341) (width 0.254) (layer "F.Cu") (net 5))
 (segment (start 150.4467 108.2341) (end 150.4467 109.2946) (width 0.254) (layer "F.Cu") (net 5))
 (segment (start 150.4467 109.2946) (end 150.0641 109.6772) (width 0.254) (layer "F.Cu") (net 5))
 (segment (start 150.0641 109.6772) (end 150.0133 109.728) (width 0.254) (layer "F.Cu") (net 5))
 (segment (start 150.0133 109.728) (end 148.9329 109.728) (width 0.254) (layer "F.Cu") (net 5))
 (segment (start 152.1841 107.315) (end 152.3467 107.4776) (width 0.254) (layer "F.Cu") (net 5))
 (segment (start 150.4467 107.4776) (end 150.6093 107.315) (width 0.254) (layer "F.Cu") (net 5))
 (via (at 148.9329 109.728) (size 0.7366) (drill 0.381) (layers "F.Cu" "B.Cu") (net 5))
 (segment (start 146.7739 109.728) (end 148.9329 109.728) (width 0.254) (layer "B.Cu") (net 5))
 (segment (start 145.9865 99.4664) (end 147.2311 99.4664) (width 0.254) (layer "B.Cu") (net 5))
 (segment (start 145.9865 108.9406) (end 145.9865 99.4664) (width 0.254) (layer "B.Cu") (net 5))
 (segment (start 146.7739 109.728) (end 145.9865 108.9406) (width 0.254) (layer "B.Cu") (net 5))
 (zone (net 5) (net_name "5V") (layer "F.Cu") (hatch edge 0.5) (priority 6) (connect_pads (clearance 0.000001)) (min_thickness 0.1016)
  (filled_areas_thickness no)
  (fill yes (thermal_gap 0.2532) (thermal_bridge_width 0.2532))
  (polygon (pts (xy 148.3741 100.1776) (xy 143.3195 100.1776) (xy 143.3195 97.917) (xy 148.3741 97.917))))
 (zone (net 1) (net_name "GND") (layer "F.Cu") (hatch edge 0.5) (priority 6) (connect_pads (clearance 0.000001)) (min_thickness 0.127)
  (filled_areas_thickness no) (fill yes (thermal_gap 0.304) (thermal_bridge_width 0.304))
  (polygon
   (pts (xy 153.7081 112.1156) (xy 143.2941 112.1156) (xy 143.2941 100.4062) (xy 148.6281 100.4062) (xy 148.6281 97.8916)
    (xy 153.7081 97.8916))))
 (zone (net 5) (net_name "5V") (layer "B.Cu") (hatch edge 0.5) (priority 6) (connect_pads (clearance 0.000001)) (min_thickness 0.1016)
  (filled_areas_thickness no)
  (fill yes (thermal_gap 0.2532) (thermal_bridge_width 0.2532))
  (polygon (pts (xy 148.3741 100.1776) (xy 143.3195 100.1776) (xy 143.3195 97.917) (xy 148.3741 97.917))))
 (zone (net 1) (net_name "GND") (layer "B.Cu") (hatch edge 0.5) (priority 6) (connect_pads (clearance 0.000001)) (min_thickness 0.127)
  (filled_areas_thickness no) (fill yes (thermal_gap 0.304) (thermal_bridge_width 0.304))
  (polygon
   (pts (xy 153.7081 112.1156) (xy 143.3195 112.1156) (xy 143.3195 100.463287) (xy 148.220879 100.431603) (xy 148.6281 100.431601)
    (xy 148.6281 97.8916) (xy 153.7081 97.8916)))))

